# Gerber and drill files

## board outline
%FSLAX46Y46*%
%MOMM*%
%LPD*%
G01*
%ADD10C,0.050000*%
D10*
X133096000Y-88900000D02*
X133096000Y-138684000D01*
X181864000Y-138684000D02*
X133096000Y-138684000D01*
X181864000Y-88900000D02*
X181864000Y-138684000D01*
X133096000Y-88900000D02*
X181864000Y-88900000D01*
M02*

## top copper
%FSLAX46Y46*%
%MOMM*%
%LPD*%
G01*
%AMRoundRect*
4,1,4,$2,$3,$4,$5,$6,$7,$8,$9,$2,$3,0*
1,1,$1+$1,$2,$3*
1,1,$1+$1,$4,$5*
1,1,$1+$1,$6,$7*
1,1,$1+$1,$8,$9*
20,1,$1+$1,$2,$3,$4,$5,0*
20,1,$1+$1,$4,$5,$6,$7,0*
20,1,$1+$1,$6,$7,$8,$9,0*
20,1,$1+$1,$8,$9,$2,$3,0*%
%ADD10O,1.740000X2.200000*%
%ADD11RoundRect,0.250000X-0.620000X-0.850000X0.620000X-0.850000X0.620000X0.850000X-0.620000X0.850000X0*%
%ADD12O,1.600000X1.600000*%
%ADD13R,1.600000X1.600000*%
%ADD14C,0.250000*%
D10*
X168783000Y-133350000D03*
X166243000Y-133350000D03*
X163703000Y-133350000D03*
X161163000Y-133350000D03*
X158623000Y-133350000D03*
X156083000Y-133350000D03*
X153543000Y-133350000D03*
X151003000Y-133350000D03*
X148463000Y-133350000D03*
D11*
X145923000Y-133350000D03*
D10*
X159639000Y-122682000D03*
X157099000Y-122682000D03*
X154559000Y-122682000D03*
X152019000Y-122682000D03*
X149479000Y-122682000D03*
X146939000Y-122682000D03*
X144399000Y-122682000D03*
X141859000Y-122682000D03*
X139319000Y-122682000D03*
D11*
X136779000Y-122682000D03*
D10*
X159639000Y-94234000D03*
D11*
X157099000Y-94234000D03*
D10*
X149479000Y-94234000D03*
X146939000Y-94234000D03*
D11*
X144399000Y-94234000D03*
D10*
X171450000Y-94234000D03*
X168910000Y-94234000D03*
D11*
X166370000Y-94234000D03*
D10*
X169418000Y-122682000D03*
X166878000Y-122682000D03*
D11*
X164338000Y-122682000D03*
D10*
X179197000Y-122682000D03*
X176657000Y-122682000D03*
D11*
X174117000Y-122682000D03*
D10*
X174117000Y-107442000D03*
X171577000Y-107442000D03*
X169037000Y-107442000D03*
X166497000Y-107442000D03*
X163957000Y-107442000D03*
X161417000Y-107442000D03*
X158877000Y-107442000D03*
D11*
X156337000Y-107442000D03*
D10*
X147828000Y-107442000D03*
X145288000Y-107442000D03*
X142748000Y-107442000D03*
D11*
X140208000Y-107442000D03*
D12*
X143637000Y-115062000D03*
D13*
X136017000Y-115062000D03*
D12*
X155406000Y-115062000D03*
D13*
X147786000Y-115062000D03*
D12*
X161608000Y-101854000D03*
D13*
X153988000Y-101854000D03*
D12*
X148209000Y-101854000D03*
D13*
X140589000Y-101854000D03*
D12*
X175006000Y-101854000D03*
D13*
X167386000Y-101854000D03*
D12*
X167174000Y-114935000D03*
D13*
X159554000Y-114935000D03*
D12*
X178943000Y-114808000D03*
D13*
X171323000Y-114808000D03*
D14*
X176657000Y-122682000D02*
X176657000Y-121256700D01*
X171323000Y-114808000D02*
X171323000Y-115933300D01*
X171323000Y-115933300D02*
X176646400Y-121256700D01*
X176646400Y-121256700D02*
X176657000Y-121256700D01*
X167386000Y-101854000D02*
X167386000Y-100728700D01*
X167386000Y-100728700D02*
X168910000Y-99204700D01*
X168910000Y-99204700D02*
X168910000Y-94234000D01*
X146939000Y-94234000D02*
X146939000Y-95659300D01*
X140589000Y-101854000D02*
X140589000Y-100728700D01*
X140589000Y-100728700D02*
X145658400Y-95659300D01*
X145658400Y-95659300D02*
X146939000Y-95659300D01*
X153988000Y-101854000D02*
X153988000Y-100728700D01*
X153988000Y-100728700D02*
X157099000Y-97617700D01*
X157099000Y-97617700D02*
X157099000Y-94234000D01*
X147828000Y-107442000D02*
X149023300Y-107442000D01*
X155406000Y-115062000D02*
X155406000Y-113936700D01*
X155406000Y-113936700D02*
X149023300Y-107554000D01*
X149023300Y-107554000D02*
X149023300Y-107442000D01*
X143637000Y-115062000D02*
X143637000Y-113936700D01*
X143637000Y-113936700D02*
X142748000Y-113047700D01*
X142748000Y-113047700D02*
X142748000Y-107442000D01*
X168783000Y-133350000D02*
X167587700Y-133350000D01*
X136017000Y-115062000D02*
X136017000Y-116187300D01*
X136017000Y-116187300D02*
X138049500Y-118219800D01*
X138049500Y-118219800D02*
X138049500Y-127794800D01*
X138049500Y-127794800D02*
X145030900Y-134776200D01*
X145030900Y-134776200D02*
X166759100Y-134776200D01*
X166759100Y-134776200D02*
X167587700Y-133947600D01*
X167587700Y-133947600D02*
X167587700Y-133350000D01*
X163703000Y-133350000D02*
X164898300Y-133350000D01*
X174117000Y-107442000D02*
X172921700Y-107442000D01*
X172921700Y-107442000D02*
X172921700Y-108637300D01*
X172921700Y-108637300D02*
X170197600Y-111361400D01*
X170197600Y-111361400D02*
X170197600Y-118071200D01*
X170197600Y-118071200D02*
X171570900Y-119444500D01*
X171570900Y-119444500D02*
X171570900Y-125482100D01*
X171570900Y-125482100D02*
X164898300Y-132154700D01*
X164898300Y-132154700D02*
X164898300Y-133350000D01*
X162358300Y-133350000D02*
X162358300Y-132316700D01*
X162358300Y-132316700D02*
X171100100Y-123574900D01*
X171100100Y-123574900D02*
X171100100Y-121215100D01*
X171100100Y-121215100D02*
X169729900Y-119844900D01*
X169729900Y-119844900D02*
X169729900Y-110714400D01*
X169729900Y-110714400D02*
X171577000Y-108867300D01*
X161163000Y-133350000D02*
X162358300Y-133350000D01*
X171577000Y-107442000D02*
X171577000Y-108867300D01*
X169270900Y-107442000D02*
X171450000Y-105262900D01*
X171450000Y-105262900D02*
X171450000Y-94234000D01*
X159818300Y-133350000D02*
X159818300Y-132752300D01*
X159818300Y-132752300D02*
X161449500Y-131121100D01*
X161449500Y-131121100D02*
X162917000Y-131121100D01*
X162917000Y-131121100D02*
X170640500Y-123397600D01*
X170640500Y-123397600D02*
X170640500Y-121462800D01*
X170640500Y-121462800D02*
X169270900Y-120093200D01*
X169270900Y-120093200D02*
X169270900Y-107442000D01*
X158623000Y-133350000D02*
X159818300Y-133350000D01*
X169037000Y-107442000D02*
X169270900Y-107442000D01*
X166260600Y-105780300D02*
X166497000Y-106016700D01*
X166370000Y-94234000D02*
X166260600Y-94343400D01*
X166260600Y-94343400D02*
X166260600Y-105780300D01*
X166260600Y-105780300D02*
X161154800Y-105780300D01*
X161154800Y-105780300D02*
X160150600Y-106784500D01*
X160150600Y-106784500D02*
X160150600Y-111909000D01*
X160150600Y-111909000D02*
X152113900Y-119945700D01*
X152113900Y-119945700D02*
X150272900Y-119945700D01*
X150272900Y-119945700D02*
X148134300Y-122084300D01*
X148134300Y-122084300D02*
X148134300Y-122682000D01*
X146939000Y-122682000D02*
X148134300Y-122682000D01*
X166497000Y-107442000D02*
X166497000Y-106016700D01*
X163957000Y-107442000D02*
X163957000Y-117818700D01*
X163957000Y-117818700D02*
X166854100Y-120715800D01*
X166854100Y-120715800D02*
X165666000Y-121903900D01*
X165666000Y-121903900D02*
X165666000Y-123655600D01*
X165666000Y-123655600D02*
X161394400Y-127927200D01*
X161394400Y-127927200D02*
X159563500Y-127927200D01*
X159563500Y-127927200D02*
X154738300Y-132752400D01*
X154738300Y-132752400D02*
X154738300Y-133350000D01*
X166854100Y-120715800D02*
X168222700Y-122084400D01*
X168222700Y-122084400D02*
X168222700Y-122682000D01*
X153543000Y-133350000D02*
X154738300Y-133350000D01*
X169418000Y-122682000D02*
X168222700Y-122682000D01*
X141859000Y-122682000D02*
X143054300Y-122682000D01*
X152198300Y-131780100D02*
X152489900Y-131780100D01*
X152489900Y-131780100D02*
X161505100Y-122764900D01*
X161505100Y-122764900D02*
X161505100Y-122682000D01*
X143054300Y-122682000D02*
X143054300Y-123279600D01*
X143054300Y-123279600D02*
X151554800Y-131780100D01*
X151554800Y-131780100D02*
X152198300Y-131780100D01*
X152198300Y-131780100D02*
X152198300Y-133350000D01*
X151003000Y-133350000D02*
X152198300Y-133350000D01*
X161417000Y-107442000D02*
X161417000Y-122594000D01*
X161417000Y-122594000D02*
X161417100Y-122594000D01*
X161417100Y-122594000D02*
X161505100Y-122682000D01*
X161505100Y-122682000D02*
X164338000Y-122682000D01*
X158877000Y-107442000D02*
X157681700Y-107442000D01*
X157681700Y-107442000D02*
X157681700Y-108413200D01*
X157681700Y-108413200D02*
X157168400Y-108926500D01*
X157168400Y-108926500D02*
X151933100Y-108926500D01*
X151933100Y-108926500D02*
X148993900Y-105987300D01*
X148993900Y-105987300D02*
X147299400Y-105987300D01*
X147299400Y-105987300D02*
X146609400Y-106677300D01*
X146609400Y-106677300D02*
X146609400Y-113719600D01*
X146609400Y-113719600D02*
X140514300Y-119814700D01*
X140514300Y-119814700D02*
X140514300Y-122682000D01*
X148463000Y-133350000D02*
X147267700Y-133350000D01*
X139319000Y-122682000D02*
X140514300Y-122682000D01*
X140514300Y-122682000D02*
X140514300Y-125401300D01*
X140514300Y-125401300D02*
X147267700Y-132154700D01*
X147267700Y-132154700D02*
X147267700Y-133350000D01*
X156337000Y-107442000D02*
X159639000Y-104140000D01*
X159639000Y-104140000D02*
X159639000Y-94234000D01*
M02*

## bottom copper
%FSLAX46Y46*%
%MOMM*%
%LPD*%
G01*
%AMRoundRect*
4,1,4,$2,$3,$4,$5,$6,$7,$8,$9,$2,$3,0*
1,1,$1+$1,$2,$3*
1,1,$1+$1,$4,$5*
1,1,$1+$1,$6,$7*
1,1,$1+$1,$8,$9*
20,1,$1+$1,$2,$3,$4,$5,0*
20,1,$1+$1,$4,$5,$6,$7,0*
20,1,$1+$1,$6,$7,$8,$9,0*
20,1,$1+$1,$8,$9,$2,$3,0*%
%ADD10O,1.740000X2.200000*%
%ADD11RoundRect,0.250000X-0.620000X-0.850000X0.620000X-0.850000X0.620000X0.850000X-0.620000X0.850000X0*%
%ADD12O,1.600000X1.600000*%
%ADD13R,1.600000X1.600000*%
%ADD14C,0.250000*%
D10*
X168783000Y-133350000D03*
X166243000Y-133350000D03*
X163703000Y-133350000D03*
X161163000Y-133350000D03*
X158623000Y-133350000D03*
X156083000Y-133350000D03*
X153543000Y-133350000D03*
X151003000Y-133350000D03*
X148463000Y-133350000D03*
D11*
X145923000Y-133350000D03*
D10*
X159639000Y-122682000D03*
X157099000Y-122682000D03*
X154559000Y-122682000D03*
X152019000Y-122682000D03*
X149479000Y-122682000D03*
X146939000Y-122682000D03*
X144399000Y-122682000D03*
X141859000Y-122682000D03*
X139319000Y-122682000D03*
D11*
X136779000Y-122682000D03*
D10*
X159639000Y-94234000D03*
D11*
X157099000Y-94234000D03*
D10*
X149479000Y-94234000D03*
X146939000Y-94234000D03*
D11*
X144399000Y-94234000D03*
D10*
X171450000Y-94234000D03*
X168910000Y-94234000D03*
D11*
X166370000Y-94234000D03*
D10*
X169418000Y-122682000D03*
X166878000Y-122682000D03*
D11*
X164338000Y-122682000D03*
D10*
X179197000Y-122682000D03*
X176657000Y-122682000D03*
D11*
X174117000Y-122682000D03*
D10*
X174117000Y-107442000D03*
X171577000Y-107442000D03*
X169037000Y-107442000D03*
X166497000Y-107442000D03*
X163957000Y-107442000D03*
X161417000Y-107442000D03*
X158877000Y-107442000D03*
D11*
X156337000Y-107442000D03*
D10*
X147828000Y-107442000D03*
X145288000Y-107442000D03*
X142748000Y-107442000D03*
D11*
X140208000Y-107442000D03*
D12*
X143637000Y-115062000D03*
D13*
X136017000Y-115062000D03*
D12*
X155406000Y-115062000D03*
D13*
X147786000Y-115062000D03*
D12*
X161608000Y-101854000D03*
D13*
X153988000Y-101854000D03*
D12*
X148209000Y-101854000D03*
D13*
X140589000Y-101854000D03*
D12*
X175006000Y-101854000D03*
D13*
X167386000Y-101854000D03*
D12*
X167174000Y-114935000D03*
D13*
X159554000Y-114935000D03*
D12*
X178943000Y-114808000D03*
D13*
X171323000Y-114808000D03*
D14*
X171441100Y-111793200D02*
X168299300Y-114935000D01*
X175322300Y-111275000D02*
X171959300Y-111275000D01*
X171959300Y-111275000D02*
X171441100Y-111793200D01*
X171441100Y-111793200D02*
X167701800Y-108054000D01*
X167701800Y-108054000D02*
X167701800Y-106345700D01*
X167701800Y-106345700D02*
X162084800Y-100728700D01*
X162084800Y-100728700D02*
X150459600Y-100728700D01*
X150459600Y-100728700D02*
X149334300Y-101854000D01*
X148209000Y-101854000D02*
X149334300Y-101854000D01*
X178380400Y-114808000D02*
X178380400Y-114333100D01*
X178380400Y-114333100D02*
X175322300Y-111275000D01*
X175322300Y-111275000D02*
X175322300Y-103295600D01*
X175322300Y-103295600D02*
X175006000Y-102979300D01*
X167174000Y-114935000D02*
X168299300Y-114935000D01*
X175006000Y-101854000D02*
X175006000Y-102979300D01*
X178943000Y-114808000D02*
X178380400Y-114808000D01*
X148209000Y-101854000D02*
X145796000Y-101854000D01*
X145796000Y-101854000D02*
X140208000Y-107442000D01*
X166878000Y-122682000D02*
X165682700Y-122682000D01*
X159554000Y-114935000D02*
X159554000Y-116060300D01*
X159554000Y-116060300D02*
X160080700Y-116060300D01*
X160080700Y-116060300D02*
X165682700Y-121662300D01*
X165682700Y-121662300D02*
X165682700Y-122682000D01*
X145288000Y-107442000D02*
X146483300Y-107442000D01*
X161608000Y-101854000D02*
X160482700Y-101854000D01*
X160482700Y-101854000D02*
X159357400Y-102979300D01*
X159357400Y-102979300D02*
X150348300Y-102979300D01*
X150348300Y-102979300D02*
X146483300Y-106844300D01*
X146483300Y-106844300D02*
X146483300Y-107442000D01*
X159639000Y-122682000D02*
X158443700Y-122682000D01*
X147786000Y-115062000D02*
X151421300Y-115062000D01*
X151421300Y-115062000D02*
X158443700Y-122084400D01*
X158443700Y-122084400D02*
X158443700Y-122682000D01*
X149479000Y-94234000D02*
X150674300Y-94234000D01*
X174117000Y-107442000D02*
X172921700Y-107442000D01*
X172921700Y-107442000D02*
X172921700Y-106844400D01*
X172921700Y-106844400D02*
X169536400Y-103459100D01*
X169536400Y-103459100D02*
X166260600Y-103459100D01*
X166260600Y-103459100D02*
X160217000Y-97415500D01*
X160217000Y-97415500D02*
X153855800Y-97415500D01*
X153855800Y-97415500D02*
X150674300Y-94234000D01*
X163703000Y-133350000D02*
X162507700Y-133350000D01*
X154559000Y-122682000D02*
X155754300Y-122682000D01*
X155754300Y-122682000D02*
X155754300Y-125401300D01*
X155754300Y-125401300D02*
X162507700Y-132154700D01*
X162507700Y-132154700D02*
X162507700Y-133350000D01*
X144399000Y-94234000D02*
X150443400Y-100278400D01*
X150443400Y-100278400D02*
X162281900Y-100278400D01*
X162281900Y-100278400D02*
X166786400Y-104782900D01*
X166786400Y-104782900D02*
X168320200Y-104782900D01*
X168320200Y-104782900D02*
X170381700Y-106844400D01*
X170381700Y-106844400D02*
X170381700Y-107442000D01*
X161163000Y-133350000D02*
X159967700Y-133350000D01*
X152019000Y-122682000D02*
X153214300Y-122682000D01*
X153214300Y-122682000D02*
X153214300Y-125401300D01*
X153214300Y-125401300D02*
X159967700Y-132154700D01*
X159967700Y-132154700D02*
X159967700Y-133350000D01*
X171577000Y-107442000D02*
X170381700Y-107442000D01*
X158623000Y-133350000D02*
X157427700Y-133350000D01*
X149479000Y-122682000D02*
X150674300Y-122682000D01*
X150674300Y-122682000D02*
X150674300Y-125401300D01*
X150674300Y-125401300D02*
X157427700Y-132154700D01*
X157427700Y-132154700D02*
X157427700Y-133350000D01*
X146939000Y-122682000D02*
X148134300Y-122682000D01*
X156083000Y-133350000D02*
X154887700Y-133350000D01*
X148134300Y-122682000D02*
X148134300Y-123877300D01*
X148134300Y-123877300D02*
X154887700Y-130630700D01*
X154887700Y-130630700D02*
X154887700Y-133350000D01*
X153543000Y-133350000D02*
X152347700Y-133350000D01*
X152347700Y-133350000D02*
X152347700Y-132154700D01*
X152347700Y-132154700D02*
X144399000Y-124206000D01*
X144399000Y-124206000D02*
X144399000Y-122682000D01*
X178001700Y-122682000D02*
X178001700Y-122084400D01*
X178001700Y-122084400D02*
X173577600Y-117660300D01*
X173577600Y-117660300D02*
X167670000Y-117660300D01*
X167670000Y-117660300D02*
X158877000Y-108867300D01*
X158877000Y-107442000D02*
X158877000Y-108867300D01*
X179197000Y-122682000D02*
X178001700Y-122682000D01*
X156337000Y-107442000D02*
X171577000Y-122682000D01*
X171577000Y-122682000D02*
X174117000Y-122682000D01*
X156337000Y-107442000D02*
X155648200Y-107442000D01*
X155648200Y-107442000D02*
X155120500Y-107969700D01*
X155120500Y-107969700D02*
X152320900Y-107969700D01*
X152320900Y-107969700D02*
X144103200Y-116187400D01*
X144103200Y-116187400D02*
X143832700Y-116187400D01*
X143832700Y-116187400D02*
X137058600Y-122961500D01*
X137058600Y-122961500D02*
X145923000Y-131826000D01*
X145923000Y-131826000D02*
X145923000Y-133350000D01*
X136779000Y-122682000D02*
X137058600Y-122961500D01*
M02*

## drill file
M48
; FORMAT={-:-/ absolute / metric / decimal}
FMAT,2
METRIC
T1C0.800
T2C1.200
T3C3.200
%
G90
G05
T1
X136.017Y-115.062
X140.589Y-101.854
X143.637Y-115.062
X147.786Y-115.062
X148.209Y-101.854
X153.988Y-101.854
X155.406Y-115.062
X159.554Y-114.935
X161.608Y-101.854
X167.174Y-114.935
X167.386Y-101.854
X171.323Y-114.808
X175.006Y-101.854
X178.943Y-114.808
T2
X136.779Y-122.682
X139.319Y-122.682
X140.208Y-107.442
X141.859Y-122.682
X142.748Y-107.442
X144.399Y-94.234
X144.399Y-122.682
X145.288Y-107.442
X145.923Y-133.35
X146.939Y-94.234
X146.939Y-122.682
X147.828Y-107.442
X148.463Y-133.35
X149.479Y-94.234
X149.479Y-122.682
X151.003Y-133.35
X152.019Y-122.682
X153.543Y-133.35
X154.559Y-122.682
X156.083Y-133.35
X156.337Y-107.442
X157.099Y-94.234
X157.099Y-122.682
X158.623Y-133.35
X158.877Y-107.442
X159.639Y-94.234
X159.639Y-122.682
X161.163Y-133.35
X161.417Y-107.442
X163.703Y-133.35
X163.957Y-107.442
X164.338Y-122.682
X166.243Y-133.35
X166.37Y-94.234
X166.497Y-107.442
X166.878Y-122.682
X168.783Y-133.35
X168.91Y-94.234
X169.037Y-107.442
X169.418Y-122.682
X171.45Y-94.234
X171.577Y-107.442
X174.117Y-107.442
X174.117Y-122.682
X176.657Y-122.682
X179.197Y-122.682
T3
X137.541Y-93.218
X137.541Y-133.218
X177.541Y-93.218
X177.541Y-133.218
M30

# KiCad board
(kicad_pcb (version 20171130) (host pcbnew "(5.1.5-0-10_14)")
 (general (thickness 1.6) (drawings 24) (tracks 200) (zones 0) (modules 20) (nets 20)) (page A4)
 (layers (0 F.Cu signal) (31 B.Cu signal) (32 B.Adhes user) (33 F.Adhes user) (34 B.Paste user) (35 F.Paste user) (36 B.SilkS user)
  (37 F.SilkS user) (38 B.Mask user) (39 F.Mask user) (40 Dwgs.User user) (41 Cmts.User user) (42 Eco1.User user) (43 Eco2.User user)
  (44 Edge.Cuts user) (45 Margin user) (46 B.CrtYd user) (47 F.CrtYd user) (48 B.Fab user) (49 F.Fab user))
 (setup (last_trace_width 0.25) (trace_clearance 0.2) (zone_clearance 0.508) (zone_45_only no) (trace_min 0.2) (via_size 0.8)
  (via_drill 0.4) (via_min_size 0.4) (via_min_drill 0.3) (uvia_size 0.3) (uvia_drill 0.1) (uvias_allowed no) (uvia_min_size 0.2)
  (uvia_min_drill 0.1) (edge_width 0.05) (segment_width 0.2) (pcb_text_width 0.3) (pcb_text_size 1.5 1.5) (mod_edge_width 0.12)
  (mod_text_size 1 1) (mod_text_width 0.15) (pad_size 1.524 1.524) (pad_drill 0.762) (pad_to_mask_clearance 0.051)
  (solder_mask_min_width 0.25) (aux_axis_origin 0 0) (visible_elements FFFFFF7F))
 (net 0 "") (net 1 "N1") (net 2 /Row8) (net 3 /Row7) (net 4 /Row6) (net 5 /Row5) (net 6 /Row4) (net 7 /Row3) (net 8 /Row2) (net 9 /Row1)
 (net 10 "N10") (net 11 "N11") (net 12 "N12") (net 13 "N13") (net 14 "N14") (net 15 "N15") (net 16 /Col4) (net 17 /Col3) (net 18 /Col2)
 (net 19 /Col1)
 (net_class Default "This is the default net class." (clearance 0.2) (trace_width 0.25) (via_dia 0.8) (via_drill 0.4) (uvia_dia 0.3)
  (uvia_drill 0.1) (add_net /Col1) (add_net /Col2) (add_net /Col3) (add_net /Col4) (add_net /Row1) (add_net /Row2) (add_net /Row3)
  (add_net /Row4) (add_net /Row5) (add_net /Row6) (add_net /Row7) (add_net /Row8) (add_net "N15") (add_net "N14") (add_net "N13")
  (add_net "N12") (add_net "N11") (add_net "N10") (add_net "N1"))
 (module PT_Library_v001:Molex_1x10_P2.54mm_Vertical (layer F.Cu) (at 145.923 133.35)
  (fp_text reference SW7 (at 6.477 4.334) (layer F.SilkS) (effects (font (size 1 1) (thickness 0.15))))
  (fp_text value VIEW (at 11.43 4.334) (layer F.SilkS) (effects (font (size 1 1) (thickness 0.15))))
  (pad 10 thru_hole oval (at 22.86 0) (size 1.74 2.2) (drill 1.2) (layers *.Cu *.Mask) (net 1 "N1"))
  (pad 9 thru_hole oval (at 20.32 0) (size 1.74 2.2) (drill 1.2) (layers *.Cu *.Mask))
  (pad 8 thru_hole oval (at 17.78 0) (size 1.74 2.2) (drill 1.2) (layers *.Cu *.Mask) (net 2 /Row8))
  (pad 7 thru_hole oval (at 15.24 0) (size 1.74 2.2) (drill 1.2) (layers *.Cu *.Mask) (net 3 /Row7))
  (pad 6 thru_hole oval (at 12.7 0) (size 1.74 2.2) (drill 1.2) (layers *.Cu *.Mask) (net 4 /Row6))
  (pad 5 thru_hole oval (at 10.16 0) (size 1.74 2.2) (drill 1.2) (layers *.Cu *.Mask) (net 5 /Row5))
  (pad 4 thru_hole oval (at 7.62 0) (size 1.74 2.2) (drill 1.2) (layers *.Cu *.Mask) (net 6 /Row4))
  (pad 3 thru_hole oval (at 5.08 0) (size 1.74 2.2) (drill 1.2) (layers *.Cu *.Mask) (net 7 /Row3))
  (pad 2 thru_hole oval (at 2.54 0) (size 1.74 2.2) (drill 1.2) (layers *.Cu *.Mask) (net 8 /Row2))
  (pad 1 thru_hole roundrect (at 0 0) (size 1.74 2.2) (drill 1.2) (layers *.Cu *.Mask) (roundrect_rratio 0.143678) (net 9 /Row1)))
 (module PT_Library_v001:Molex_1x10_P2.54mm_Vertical (layer F.Cu) (at 136.779 122.682)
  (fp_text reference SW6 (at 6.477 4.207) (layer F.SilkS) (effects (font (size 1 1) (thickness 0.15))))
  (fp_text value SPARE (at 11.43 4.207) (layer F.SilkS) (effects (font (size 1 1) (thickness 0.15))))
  (pad 10 thru_hole oval (at 22.86 0) (size 1.74 2.2) (drill 1.2) (layers *.Cu *.Mask) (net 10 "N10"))
  (pad 9 thru_hole oval (at 20.32 0) (size 1.74 2.2) (drill 1.2) (layers *.Cu *.Mask))
  (pad 8 thru_hole oval (at 17.78 0) (size 1.74 2.2) (drill 1.2) (layers *.Cu *.Mask) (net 2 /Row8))
  (pad 7 thru_hole oval (at 15.24 0) (size 1.74 2.2) (drill 1.2) (layers *.Cu *.Mask) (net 3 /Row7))
  (pad 6 thru_hole oval (at 12.7 0) (size 1.74 2.2) (drill 1.2) (layers *.Cu *.Mask) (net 4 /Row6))
  (pad 5 thru_hole oval (at 10.16 0) (size 1.74 2.2) (drill 1.2) (layers *.Cu *.Mask) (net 5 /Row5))
  (pad 4 thru_hole oval (at 7.62 0) (size 1.74 2.2) (drill 1.2) (layers *.Cu *.Mask) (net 6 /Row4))
  (pad 3 thru_hole oval (at 5.08 0) (size 1.74 2.2) (drill 1.2) (layers *.Cu *.Mask) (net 7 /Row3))
  (pad 2 thru_hole oval (at 2.54 0) (size 1.74 2.2) (drill 1.2) (layers *.Cu *.Mask) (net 8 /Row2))
  (pad 1 thru_hole roundrect (at 0 0) (size 1.74 2.2) (drill 1.2) (layers *.Cu *.Mask) (roundrect_rratio 0.143678) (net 9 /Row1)))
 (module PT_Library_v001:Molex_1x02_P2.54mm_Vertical (layer F.Cu) (at 157.099 94.234)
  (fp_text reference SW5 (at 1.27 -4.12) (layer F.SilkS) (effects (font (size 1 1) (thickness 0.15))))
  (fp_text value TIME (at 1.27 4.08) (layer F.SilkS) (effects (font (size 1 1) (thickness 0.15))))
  (pad 2 thru_hole oval (at 2.54 0) (size 1.74 2.2) (drill 1.2) (layers *.Cu *.Mask) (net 9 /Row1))
  (pad 1 thru_hole roundrect (at 0 0) (size 1.74 2.2) (drill 1.2) (layers *.Cu *.Mask) (roundrect_rratio 0.143678) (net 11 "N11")))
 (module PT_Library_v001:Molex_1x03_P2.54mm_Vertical (layer F.Cu) (at 144.399 94.234)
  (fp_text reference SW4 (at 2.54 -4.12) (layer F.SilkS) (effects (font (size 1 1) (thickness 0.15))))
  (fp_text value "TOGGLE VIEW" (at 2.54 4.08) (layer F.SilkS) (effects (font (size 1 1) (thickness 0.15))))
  (pad 3 thru_hole oval (at 5.08 0) (size 1.74 2.2) (drill 1.2) (layers *.Cu *.Mask) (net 2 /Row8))
  (pad 2 thru_hole oval (at 2.54 0) (size 1.74 2.2) (drill 1.2) (layers *.Cu *.Mask) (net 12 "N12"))
  (pad 1 thru_hole roundrect (at 0 0) (size 1.74 2.2) (drill 1.2) (layers *.Cu *.Mask) (roundrect_rratio 0.143678) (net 3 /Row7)))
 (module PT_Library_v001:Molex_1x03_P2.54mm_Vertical (layer F.Cu) (at 166.37 94.234)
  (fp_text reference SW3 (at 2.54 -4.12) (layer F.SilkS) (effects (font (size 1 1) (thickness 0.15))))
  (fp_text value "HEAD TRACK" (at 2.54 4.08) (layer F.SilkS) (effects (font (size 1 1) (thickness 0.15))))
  (pad 3 thru_hole oval (at 5.08 0) (size 1.74 2.2) (drill 1.2) (layers *.Cu *.Mask) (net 4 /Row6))
  (pad 2 thru_hole oval (at 2.54 0) (size 1.74 2.2) (drill 1.2) (layers *.Cu *.Mask) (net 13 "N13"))
  (pad 1 thru_hole roundrect (at 0 0) (size 1.74 2.2) (drill 1.2) (layers *.Cu *.Mask) (roundrect_rratio 0.143678) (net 5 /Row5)))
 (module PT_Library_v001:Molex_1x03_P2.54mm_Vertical (layer F.Cu) (at 164.338 122.682)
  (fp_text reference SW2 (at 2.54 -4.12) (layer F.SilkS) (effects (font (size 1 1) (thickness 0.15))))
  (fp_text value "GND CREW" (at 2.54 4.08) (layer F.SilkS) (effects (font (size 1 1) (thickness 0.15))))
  (pad 3 thru_hole oval (at 5.08 0) (size 1.74 2.2) (drill 1.2) (layers *.Cu *.Mask) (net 6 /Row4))
  (pad 2 thru_hole oval (at 2.54 0) (size 1.74 2.2) (drill 1.2) (layers *.Cu *.Mask) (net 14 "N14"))
  (pad 1 thru_hole roundrect (at 0 0) (size 1.74 2.2) (drill 1.2) (layers *.Cu *.Mask) (roundrect_rratio 0.143678) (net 7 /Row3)))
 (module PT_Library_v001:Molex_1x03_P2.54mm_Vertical (layer F.Cu) (at 174.117 122.682)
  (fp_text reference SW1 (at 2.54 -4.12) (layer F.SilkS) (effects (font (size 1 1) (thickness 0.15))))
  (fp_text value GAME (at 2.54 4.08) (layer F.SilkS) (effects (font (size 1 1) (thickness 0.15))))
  (pad 3 thru_hole oval (at 5.08 0) (size 1.74 2.2) (drill 1.2) (layers *.Cu *.Mask) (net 8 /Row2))
  (pad 2 thru_hole oval (at 2.54 0) (size 1.74 2.2) (drill 1.2) (layers *.Cu *.Mask) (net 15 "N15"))
  (pad 1 thru_hole roundrect (at 0 0) (size 1.74 2.2) (drill 1.2) (layers *.Cu *.Mask) (roundrect_rratio 0.143678) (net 9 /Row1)))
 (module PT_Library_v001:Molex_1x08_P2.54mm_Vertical (layer F.Cu) (at 156.337 107.442)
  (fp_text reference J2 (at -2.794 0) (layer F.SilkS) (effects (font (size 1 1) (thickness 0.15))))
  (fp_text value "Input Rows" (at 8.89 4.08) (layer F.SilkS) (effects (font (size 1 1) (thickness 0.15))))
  (pad 8 thru_hole oval (at 17.78 0) (size 1.74 2.2) (drill 1.2) (layers *.Cu *.Mask) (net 2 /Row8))
  (pad 7 thru_hole oval (at 15.24 0) (size 1.74 2.2) (drill 1.2) (layers *.Cu *.Mask) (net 3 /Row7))
  (pad 6 thru_hole oval (at 12.7 0) (size 1.74 2.2) (drill 1.2) (layers *.Cu *.Mask) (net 4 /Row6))
  (pad 5 thru_hole oval (at 10.16 0) (size 1.74 2.2) (drill 1.2) (layers *.Cu *.Mask) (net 5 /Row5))
  (pad 4 thru_hole oval (at 7.62 0) (size 1.74 2.2) (drill 1.2) (layers *.Cu *.Mask) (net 6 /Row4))
  (pad 3 thru_hole oval (at 5.08 0) (size 1.74 2.2) (drill 1.2) (layers *.Cu *.Mask) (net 7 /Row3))
  (pad 2 thru_hole oval (at 2.54 0) (size 1.74 2.2) (drill 1.2) (layers *.Cu *.Mask) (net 8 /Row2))
  (pad 1 thru_hole roundrect (at 0 0) (size 1.74 2.2) (drill 1.2) (layers *.Cu *.Mask) (roundrect_rratio 0.143678) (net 9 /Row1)))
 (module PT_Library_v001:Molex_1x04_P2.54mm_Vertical (layer F.Cu) (at 140.208 107.442)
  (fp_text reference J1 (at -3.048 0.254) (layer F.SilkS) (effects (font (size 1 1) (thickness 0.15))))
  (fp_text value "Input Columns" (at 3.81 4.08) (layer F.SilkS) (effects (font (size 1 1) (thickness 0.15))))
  (pad 4 thru_hole oval (at 7.62 0) (size 1.74 2.2) (drill 1.2) (layers *.Cu *.Mask) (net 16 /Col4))
  (pad 3 thru_hole oval (at 5.08 0) (size 1.74 2.2) (drill 1.2) (layers *.Cu *.Mask) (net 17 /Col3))
  (pad 2 thru_hole oval (at 2.54 0) (size 1.74 2.2) (drill 1.2) (layers *.Cu *.Mask) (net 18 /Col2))
  (pad 1 thru_hole roundrect (at 0 0) (size 1.74 2.2) (drill 1.2) (layers *.Cu *.Mask) (roundrect_rratio 0.143678) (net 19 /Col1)))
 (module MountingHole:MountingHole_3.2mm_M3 (layer F.Cu) (at 137.541 93.218)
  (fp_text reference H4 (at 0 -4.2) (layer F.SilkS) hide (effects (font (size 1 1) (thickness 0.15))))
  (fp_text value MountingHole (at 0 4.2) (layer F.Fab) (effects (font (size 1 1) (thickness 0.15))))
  (pad 1 np_thru_hole circle (at 0 0) (size 3.2 3.2) (drill 3.2) (layers *.Cu *.Mask)))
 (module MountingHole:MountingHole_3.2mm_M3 (layer F.Cu) (at 177.541 93.218)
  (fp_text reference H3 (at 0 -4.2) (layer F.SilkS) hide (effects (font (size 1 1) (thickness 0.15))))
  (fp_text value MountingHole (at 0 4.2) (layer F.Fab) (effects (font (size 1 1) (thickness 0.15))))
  (pad 1 np_thru_hole circle (at 0 0) (size 3.2 3.2) (drill 3.2) (layers *.Cu *.Mask)))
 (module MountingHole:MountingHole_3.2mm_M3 (layer F.Cu) (at 137.541 133.218)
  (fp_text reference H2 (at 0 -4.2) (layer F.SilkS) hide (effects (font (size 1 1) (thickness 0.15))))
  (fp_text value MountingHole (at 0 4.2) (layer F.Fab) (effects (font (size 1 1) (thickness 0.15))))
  (pad 1 np_thru_hole circle (at 0 0) (size 3.2 3.2) (drill 3.2) (layers *.Cu *.Mask)))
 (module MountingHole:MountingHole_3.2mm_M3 (layer F.Cu) (at 177.541 133.218)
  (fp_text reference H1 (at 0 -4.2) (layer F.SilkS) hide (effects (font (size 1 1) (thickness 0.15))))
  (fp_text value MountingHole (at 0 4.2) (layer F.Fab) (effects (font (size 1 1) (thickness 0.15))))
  (pad 1 np_thru_hole circle (at 0 0) (size 3.2 3.2) (drill 3.2) (layers *.Cu *.Mask)))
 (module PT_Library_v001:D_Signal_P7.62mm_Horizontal (layer F.Cu) (at 136.017 115.062)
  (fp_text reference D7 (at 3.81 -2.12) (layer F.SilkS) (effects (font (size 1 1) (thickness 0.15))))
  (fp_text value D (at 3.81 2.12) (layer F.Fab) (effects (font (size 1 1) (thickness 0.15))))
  (pad 2 thru_hole oval (at 7.62 0) (size 1.6 1.6) (drill 0.8) (layers *.Cu *.Mask) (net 18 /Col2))
  (pad 1 thru_hole rect (at 0 0) (size 1.6 1.6) (drill 0.8) (layers *.Cu *.Mask) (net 1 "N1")))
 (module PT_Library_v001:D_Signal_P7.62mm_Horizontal (layer F.Cu) (at 147.786 115.062)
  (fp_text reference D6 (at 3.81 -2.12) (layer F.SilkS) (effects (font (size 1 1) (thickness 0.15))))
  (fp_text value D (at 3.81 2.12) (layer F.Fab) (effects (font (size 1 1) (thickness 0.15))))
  (pad 2 thru_hole oval (at 7.62 0) (size 1.6 1.6) (drill 0.8) (layers *.Cu *.Mask) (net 16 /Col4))
  (pad 1 thru_hole rect (at 0 0) (size 1.6 1.6) (drill 0.8) (layers *.Cu *.Mask) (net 10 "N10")))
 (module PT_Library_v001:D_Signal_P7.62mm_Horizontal (layer F.Cu) (at 153.988 101.854)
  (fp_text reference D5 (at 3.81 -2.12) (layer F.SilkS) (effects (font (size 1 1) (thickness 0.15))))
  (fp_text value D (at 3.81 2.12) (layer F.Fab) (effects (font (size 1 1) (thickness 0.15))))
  (pad 2 thru_hole oval (at 7.62 0) (size 1.6 1.6) (drill 0.8) (layers *.Cu *.Mask) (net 17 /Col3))
  (pad 1 thru_hole rect (at 0 0) (size 1.6 1.6) (drill 0.8) (layers *.Cu *.Mask) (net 11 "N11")))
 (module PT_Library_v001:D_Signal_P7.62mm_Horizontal (layer F.Cu) (at 140.589 101.854)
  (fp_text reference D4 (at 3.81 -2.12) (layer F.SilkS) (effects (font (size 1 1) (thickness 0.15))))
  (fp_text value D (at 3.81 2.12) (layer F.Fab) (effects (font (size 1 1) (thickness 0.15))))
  (pad 2 thru_hole oval (at 7.62 0) (size 1.6 1.6) (drill 0.8) (layers *.Cu *.Mask) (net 19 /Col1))
  (pad 1 thru_hole rect (at 0 0) (size 1.6 1.6) (drill 0.8) (layers *.Cu *.Mask) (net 12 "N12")))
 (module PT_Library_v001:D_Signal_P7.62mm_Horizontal (layer F.Cu) (at 167.386 101.854)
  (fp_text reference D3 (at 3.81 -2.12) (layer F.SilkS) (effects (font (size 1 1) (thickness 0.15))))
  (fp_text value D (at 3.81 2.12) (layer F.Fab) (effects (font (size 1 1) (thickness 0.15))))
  (pad 2 thru_hole oval (at 7.62 0) (size 1.6 1.6) (drill 0.8) (layers *.Cu *.Mask) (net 19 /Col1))
  (pad 1 thru_hole rect (at 0 0) (size 1.6 1.6) (drill 0.8) (layers *.Cu *.Mask) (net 13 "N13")))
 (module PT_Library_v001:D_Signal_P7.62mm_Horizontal (layer F.Cu) (at 159.554 114.935)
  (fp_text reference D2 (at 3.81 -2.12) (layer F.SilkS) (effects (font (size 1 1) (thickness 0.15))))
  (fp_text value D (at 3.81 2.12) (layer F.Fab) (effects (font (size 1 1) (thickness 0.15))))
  (pad 2 thru_hole oval (at 7.62 0) (size 1.6 1.6) (drill 0.8) (layers *.Cu *.Mask) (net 19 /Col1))
  (pad 1 thru_hole rect (at 0 0) (size 1.6 1.6) (drill 0.8) (layers *.Cu *.Mask) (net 14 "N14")))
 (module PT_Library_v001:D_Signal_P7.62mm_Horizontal (layer F.Cu) (at 171.323 114.808)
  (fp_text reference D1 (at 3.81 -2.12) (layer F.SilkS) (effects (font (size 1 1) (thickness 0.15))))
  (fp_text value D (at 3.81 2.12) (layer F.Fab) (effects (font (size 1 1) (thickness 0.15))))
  (pad 2 thru_hole oval (at 7.62 0) (size 1.6 1.6) (drill 0.8) (layers *.Cu *.Mask) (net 19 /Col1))
  (pad 1 thru_hole rect (at 0 0) (size 1.6 1.6) (drill 0.8) (layers *.Cu *.Mask) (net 15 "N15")))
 (gr_line (start 133.096 88.9) (end 133.096 138.684) (layer Edge.Cuts) (width 0.05))
 (gr_line (start 181.864 138.684) (end 133.096 138.684) (layer Edge.Cuts) (width 0.05))
 (gr_line (start 181.864 88.9) (end 181.864 138.684) (layer Edge.Cuts) (width 0.05))
 (gr_line (start 133.096 88.9) (end 181.864 88.9) (layer Edge.Cuts) (width 0.05))
 (segment (start 171.4411 111.7932) (end 168.2993 114.935) (width 0.25) (layer B.Cu) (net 19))
 (segment (start 175.3223 111.275) (end 171.9593 111.275) (width 0.25) (layer B.Cu) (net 19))
 (segment (start 171.9593 111.275) (end 171.4411 111.7932) (width 0.25) (layer B.Cu) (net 19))
 (segment (start 171.4411 111.7932) (end 167.7018 108.054) (width 0.25) (layer B.Cu) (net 19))
 (segment (start 167.7018 108.054) (end 167.7018 106.3457) (width 0.25) (layer B.Cu) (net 19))
 (segment (start 167.7018 106.3457) (end 162.0848 100.7287) (width 0.25) (layer B.Cu) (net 19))
 (segment (start 162.0848 100.7287) (end 150.4596 100.7287) (width 0.25) (layer B.Cu) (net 19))
 (segment (start 150.4596 100.7287) (end 149.3343 101.854) (width 0.25) (layer B.Cu) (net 19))
 (segment (start 148.209 101.854) (end 149.3343 101.854) (width 0.25) (layer B.Cu) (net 19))
 (segment (start 178.3804 114.808) (end 178.3804 114.3331) (width 0.25) (layer B.Cu) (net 19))
 (segment (start 178.3804 114.3331) (end 175.3223 111.275) (width 0.25) (layer B.Cu) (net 19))
 (segment (start 175.3223 111.275) (end 175.3223 103.2956) (width 0.25) (layer B.Cu) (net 19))
 (segment (start 175.3223 103.2956) (end 175.006 102.9793) (width 0.25) (layer B.Cu) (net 19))
 (segment (start 167.174 114.935) (end 168.2993 114.935) (width 0.25) (layer B.Cu) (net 19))
 (segment (start 175.006 101.854) (end 175.006 102.9793) (width 0.25) (layer B.Cu) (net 19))
 (segment (start 178.943 114.808) (end 178.3804 114.808) (width 0.25) (layer B.Cu) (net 19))
 (segment (start 148.209 101.854) (end 145.796 101.854) (width 0.25) (layer B.Cu) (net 19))
 (segment (start 145.796 101.854) (end 140.208 107.442) (width 0.25) (layer B.Cu) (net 19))
 (segment (start 176.657 122.682) (end 176.657 121.2567) (width 0.25) (layer F.Cu) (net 15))
 (segment (start 171.323 114.808) (end 171.323 115.9333) (width 0.25) (layer F.Cu) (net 15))
 (segment (start 171.323 115.9333) (end 176.6464 121.2567) (width 0.25) (layer F.Cu) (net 15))
 (segment (start 176.6464 121.2567) (end 176.657 121.2567) (width 0.25) (layer F.Cu) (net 15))
 (segment (start 166.878 122.682) (end 165.6827 122.682) (width 0.25) (layer B.Cu) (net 14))
 (segment (start 159.554 114.935) (end 159.554 116.0603) (width 0.25) (layer B.Cu) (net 14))
 (segment (start 159.554 116.0603) (end 160.0807 116.0603) (width 0.25) (layer B.Cu) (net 14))
 (segment (start 160.0807 116.0603) (end 165.6827 121.6623) (width 0.25) (layer B.Cu) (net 14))
 (segment (start 165.6827 121.6623) (end 165.6827 122.682) (width 0.25) (layer B.Cu) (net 14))
 (segment (start 167.386 101.854) (end 167.386 100.7287) (width 0.25) (layer F.Cu) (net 13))
 (segment (start 167.386 100.7287) (end 168.91 99.2047) (width 0.25) (layer F.Cu) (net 13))
 (segment (start 168.91 99.2047) (end 168.91 94.234) (width 0.25) (layer F.Cu) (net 13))
 (segment (start 146.939 94.234) (end 146.939 95.6593) (width 0.25) (layer F.Cu) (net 12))
 (segment (start 140.589 101.854) (end 140.589 100.7287) (width 0.25) (layer F.Cu) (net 12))
 (segment (start 140.589 100.7287) (end 145.6584 95.6593) (width 0.25) (layer F.Cu) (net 12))
 (segment (start 145.6584 95.6593) (end 146.939 95.6593) (width 0.25) (layer F.Cu) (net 12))
 (segment (start 145.288 107.442) (end 146.4833 107.442) (width 0.25) (layer B.Cu) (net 17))
 (segment (start 161.608 101.854) (end 160.4827 101.854) (width 0.25) (layer B.Cu) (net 17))
 (segment (start 160.4827 101.854) (end 159.3574 102.9793) (width 0.25) (layer B.Cu) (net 17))
 (segment (start 159.3574 102.9793) (end 150.3483 102.9793) (width 0.25) (layer B.Cu) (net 17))
 (segment (start 150.3483 102.9793) (end 146.4833 106.8443) (width 0.25) (layer B.Cu) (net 17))
 (segment (start 146.4833 106.8443) (end 146.4833 107.442) (width 0.25) (layer B.Cu) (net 17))
 (segment (start 153.988 101.854) (end 153.988 100.7287) (width 0.25) (layer F.Cu) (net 11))
 (segment (start 153.988 100.7287) (end 157.099 97.6177) (width 0.25) (layer F.Cu) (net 11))
 (segment (start 157.099 97.6177) (end 157.099 94.234) (width 0.25) (layer F.Cu) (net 11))
 (segment (start 147.828 107.442) (end 149.0233 107.442) (width 0.25) (layer F.Cu) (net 16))
 (segment (start 155.406 115.062) (end 155.406 113.9367) (width 0.25) (layer F.Cu) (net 16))
 (segment (start 155.406 113.9367) (end 149.0233 107.554) (width 0.25) (layer F.Cu) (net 16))
 (segment (start 149.0233 107.554) (end 149.0233 107.442) (width 0.25) (layer F.Cu) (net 16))
 (segment (start 159.639 122.682) (end 158.4437 122.682) (width 0.25) (layer B.Cu) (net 10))
 (segment (start 147.786 115.062) (end 151.4213 115.062) (width 0.25) (layer B.Cu) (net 10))
 (segment (start 151.4213 115.062) (end 158.4437 122.0844) (width 0.25) (layer B.Cu) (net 10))
 (segment (start 158.4437 122.0844) (end 158.4437 122.682) (width 0.25) (layer B.Cu) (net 10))
 (segment (start 143.637 115.062) (end 143.637 113.9367) (width 0.25) (layer F.Cu) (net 18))
 (segment (start 143.637 113.9367) (end 142.748 113.0477) (width 0.25) (layer F.Cu) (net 18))
 (segment (start 142.748 113.0477) (end 142.748 107.442) (width 0.25) (layer F.Cu) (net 18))
 (segment (start 168.783 133.35) (end 167.5877 133.35) (width 0.25) (layer F.Cu) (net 1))
 (segment (start 136.017 115.062) (end 136.017 116.1873) (width 0.25) (layer F.Cu) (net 1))
 (segment (start 136.017 116.1873) (end 138.0495 118.2198) (width 0.25) (layer F.Cu) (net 1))
 (segment (start 138.0495 118.2198) (end 138.0495 127.7948) (width 0.25) (layer F.Cu) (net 1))
 (segment (start 138.0495 127.7948) (end 145.0309 134.7762) (width 0.25) (layer F.Cu) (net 1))
 (segment (start 145.0309 134.7762) (end 166.7591 134.7762) (width 0.25) (layer F.Cu) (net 1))
 (segment (start 166.7591 134.7762) (end 167.5877 133.9476) (width 0.25) (layer F.Cu) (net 1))
 (segment (start 167.5877 133.9476) (end 167.5877 133.35) (width 0.25) (layer F.Cu) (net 1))
 (segment (start 163.703 133.35) (end 164.8983 133.35) (width 0.25) (layer F.Cu) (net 2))
 (segment (start 174.117 107.442) (end 172.9217 107.442) (width 0.25) (layer F.Cu) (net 2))
 (segment (start 172.9217 107.442) (end 172.9217 108.6373) (width 0.25) (layer F.Cu) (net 2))
 (segment (start 172.9217 108.6373) (end 170.1976 111.3614) (width 0.25) (layer F.Cu) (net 2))
 (segment (start 170.1976 111.3614) (end 170.1976 118.0712) (width 0.25) (layer F.Cu) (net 2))
 (segment (start 170.1976 118.0712) (end 171.5709 119.4445) (width 0.25) (layer F.Cu) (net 2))
 (segment (start 171.5709 119.4445) (end 171.5709 125.4821) (width 0.25) (layer F.Cu) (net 2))
 (segment (start 171.5709 125.4821) (end 164.8983 132.1547) (width 0.25) (layer F.Cu) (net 2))
 (segment (start 164.8983 132.1547) (end 164.8983 133.35) (width 0.25) (layer F.Cu) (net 2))
 (segment (start 149.479 94.234) (end 150.6743 94.234) (width 0.25) (layer B.Cu) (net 2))
 (segment (start 174.117 107.442) (end 172.9217 107.442) (width 0.25) (layer B.Cu) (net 2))
 (segment (start 172.9217 107.442) (end 172.9217 106.8444) (width 0.25) (layer B.Cu) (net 2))
 (segment (start 172.9217 106.8444) (end 169.5364 103.4591) (width 0.25) (layer B.Cu) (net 2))
 (segment (start 169.5364 103.4591) (end 166.2606 103.4591) (width 0.25) (layer B.Cu) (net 2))
 (segment (start 166.2606 103.4591) (end 160.217 97.4155) (width 0.25) (layer B.Cu) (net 2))
 (segment (start 160.217 97.4155) (end 153.8558 97.4155) (width 0.25) (layer B.Cu) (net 2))
 (segment (start 153.8558 97.4155) (end 150.6743 94.234) (width 0.25) (layer B.Cu) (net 2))
 (segment (start 163.703 133.35) (end 162.5077 133.35) (width 0.25) (layer B.Cu) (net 2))
 (segment (start 154.559 122.682) (end 155.7543 122.682) (width 0.25) (layer B.Cu) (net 2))
 (segment (start 155.7543 122.682) (end 155.7543 125.4013) (width 0.25) (layer B.Cu) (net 2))
 (segment (start 155.7543 125.4013) (end 162.5077 132.1547) (width 0.25) (layer B.Cu) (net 2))
 (segment (start 162.5077 132.1547) (end 162.5077 133.35) (width 0.25) (layer B.Cu) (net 2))
 (segment (start 162.3583 133.35) (end 162.3583 132.3167) (width 0.25) (layer F.Cu) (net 3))
 (segment (start 162.3583 132.3167) (end 171.1001 123.5749) (width 0.25) (layer F.Cu) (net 3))
 (segment (start 171.1001 123.5749) (end 171.1001 121.2151) (width 0.25) (layer F.Cu) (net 3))
 (segment (start 171.1001 121.2151) (end 169.7299 119.8449) (width 0.25) (layer F.Cu) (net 3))
 (segment (start 169.7299 119.8449) (end 169.7299 110.7144) (width 0.25) (layer F.Cu) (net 3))
 (segment (start 169.7299 110.7144) (end 171.577 108.8673) (width 0.25) (layer F.Cu) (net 3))
 (segment (start 161.163 133.35) (end 162.3583 133.35) (width 0.25) (layer F.Cu) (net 3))
 (segment (start 171.577 107.442) (end 171.577 108.8673) (width 0.25) (layer F.Cu) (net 3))
 (segment (start 144.399 94.234) (end 150.4434 100.2784) (width 0.25) (layer B.Cu) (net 3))
 (segment (start 150.4434 100.2784) (end 162.2819 100.2784) (width 0.25) (layer B.Cu) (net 3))
 (segment (start 162.2819 100.2784) (end 166.7864 104.7829) (width 0.25) (layer B.Cu) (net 3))
 (segment (start 166.7864 104.7829) (end 168.3202 104.7829) (width 0.25) (layer B.Cu) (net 3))
 (segment (start 168.3202 104.7829) (end 170.3817 106.8444) (width 0.25) (layer B.Cu) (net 3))
 (segment (start 170.3817 106.8444) (end 170.3817 107.442) (width 0.25) (layer B.Cu) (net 3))
 (segment (start 161.163 133.35) (end 159.9677 133.35) (width 0.25) (layer B.Cu) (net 3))
 (segment (start 152.019 122.682) (end 153.2143 122.682) (width 0.25) (layer B.Cu) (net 3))
 (segment (start 153.2143 122.682) (end 153.2143 125.4013) (width 0.25) (layer B.Cu) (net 3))
 (segment (start 153.2143 125.4013) (end 159.9677 132.1547) (width 0.25) (layer B.Cu) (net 3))
 (segment (start 159.9677 132.1547) (end 159.9677 133.35) (width 0.25) (layer B.Cu) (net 3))
 (segment (start 171.577 107.442) (end 170.3817 107.442) (width 0.25) (layer B.Cu) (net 3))
 (segment (start 169.2709 107.442) (end 171.45 105.2629) (width 0.25) (layer F.Cu) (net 4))
 (segment (start 171.45 105.2629) (end 171.45 94.234) (width 0.25) (layer F.Cu) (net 4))
 (segment (start 159.8183 133.35) (end 159.8183 132.7523) (width 0.25) (layer F.Cu) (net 4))
 (segment (start 159.8183 132.7523) (end 161.4495 131.1211) (width 0.25) (layer F.Cu) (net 4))
 (segment (start 161.4495 131.1211) (end 162.917 131.1211) (width 0.25) (layer F.Cu) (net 4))
 (segment (start 162.917 131.1211) (end 170.6405 123.3976) (width 0.25) (layer F.Cu) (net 4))
 (segment (start 170.6405 123.3976) (end 170.6405 121.4628) (width 0.25) (layer F.Cu) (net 4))
 (segment (start 170.6405 121.4628) (end 169.2709 120.0932) (width 0.25) (layer F.Cu) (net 4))
 (segment (start 169.2709 120.0932) (end 169.2709 107.442) (width 0.25) (layer F.Cu) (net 4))
 (segment (start 158.623 133.35) (end 159.8183 133.35) (width 0.25) (layer F.Cu) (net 4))
 (segment (start 169.037 107.442) (end 169.2709 107.442) (width 0.25) (layer F.Cu) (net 4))
 (segment (start 158.623 133.35) (end 157.4277 133.35) (width 0.25) (layer B.Cu) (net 4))
 (segment (start 149.479 122.682) (end 150.6743 122.682) (width 0.25) (layer B.Cu) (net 4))
 (segment (start 150.6743 122.682) (end 150.6743 125.4013) (width 0.25) (layer B.Cu) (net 4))
 (segment (start 150.6743 125.4013) (end 157.4277 132.1547) (width 0.25) (layer B.Cu) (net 4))
 (segment (start 157.4277 132.1547) (end 157.4277 133.35) (width 0.25) (layer B.Cu) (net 4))
 (segment (start 146.939 122.682) (end 148.1343 122.682) (width 0.25) (layer B.Cu) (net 5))
 (segment (start 156.083 133.35) (end 154.8877 133.35) (width 0.25) (layer B.Cu) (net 5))
 (segment (start 148.1343 122.682) (end 148.1343 123.8773) (width 0.25) (layer B.Cu) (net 5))
 (segment (start 148.1343 123.8773) (end 154.8877 130.6307) (width 0.25) (layer B.Cu) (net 5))
 (segment (start 154.8877 130.6307) (end 154.8877 133.35) (width 0.25) (layer B.Cu) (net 5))
 (segment (start 166.2606 105.7803) (end 166.497 106.0167) (width 0.25) (layer F.Cu) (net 5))
 (segment (start 166.37 94.234) (end 166.2606 94.3434) (width 0.25) (layer F.Cu) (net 5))
 (segment (start 166.2606 94.3434) (end 166.2606 105.7803) (width 0.25) (layer F.Cu) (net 5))
 (segment (start 166.2606 105.7803) (end 161.1548 105.7803) (width 0.25) (layer F.Cu) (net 5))
 (segment (start 161.1548 105.7803) (end 160.1506 106.7845) (width 0.25) (layer F.Cu) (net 5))
 (segment (start 160.1506 106.7845) (end 160.1506 111.909) (width 0.25) (layer F.Cu) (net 5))
 (segment (start 160.1506 111.909) (end 152.1139 119.9457) (width 0.25) (layer F.Cu) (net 5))
 (segment (start 152.1139 119.9457) (end 150.2729 119.9457) (width 0.25) (layer F.Cu) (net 5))
 (segment (start 150.2729 119.9457) (end 148.1343 122.0843) (width 0.25) (layer F.Cu) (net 5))
 (segment (start 148.1343 122.0843) (end 148.1343 122.682) (width 0.25) (layer F.Cu) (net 5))
 (segment (start 146.939 122.682) (end 148.1343 122.682) (width 0.25) (layer F.Cu) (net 5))
 (segment (start 166.497 107.442) (end 166.497 106.0167) (width 0.25) (layer F.Cu) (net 5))
 (segment (start 163.957 107.442) (end 163.957 117.8187) (width 0.25) (layer F.Cu) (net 6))
 (segment (start 163.957 117.8187) (end 166.8541 120.7158) (width 0.25) (layer F.Cu) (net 6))
 (segment (start 166.8541 120.7158) (end 165.666 121.9039) (width 0.25) (layer F.Cu) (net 6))
 (segment (start 165.666 121.9039) (end 165.666 123.6556) (width 0.25) (layer F.Cu) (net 6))
 (segment (start 165.666 123.6556) (end 161.3944 127.9272) (width 0.25) (layer F.Cu) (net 6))
 (segment (start 161.3944 127.9272) (end 159.5635 127.9272) (width 0.25) (layer F.Cu) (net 6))
 (segment (start 159.5635 127.9272) (end 154.7383 132.7524) (width 0.25) (layer F.Cu) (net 6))
 (segment (start 154.7383 132.7524) (end 154.7383 133.35) (width 0.25) (layer F.Cu) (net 6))
 (segment (start 166.8541 120.7158) (end 168.2227 122.0844) (width 0.25) (layer F.Cu) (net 6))
 (segment (start 168.2227 122.0844) (end 168.2227 122.682) (width 0.25) (layer F.Cu) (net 6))
 (segment (start 153.543 133.35) (end 154.7383 133.35) (width 0.25) (layer F.Cu) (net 6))
 (segment (start 169.418 122.682) (end 168.2227 122.682) (width 0.25) (layer F.Cu) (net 6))
 (segment (start 153.543 133.35) (end 152.3477 133.35) (width 0.25) (layer B.Cu) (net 6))
 (segment (start 152.3477 133.35) (end 152.3477 132.1547) (width 0.25) (layer B.Cu) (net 6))
 (segment (start 152.3477 132.1547) (end 144.399 124.206) (width 0.25) (layer B.Cu) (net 6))
 (segment (start 144.399 124.206) (end 144.399 122.682) (width 0.25) (layer B.Cu) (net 6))
 (segment (start 141.859 122.682) (end 143.0543 122.682) (width 0.25) (layer F.Cu) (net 7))
 (segment (start 152.1983 131.7801) (end 152.4899 131.7801) (width 0.25) (layer F.Cu) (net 7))
 (segment (start 152.4899 131.7801) (end 161.5051 122.7649) (width 0.25) (layer F.Cu) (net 7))
 (segment (start 161.5051 122.7649) (end 161.5051 122.682) (width 0.25) (layer F.Cu) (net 7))
 (segment (start 143.0543 122.682) (end 143.0543 123.2796) (width 0.25) (layer F.Cu) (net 7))
 (segment (start 143.0543 123.2796) (end 151.5548 131.7801) (width 0.25) (layer F.Cu) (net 7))
 (segment (start 151.5548 131.7801) (end 152.1983 131.7801) (width 0.25) (layer F.Cu) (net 7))
 (segment (start 152.1983 131.7801) (end 152.1983 133.35) (width 0.25) (layer F.Cu) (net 7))
 (segment (start 151.003 133.35) (end 152.1983 133.35) (width 0.25) (layer F.Cu) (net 7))
 (segment (start 161.417 107.442) (end 161.417 122.594) (width 0.25) (layer F.Cu) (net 7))
 (segment (start 161.417 122.594) (end 161.4171 122.594) (width 0.25) (layer F.Cu) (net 7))
 (segment (start 161.4171 122.594) (end 161.5051 122.682) (width 0.25) (layer F.Cu) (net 7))
 (segment (start 161.5051 122.682) (end 164.338 122.682) (width 0.25) (layer F.Cu) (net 7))
 (segment (start 178.0017 122.682) (end 178.0017 122.0844) (width 0.25) (layer B.Cu) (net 8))
 (segment (start 178.0017 122.0844) (end 173.5776 117.6603) (width 0.25) (layer B.Cu) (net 8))
 (segment (start 173.5776 117.6603) (end 167.67 117.6603) (width 0.25) (layer B.Cu) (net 8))
 (segment (start 167.67 117.6603) (end 158.877 108.8673) (width 0.25) (layer B.Cu) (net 8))
 (segment (start 158.877 107.442) (end 158.877 108.8673) (width 0.25) (layer B.Cu) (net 8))
 (segment (start 179.197 122.682) (end 178.0017 122.682) (width 0.25) (layer B.Cu) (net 8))
 (segment (start 158.877 107.442) (end 157.6817 107.442) (width 0.25) (layer F.Cu) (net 8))
 (segment (start 157.6817 107.442) (end 157.6817 108.4132) (width 0.25) (layer F.Cu) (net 8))
 (segment (start 157.6817 108.4132) (end 157.1684 108.9265) (width 0.25) (layer F.Cu) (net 8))
 (segment (start 157.1684 108.9265) (end 151.9331 108.9265) (width 0.25) (layer F.Cu) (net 8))
 (segment (start 151.9331 108.9265) (end 148.9939 105.9873) (width 0.25) (layer F.Cu) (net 8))
 (segment (start 148.9939 105.9873) (end 147.2994 105.9873) (width 0.25) (layer F.Cu) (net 8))
 (segment (start 147.2994 105.9873) (end 146.6094 106.6773) (width 0.25) (layer F.Cu) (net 8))
 (segment (start 146.6094 106.6773) (end 146.6094 113.7196) (width 0.25) (layer F.Cu) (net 8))
 (segment (start 146.6094 113.7196) (end 140.5143 119.8147) (width 0.25) (layer F.Cu) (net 8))
 (segment (start 140.5143 119.8147) (end 140.5143 122.682) (width 0.25) (layer F.Cu) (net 8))
 (segment (start 148.463 133.35) (end 147.2677 133.35) (width 0.25) (layer F.Cu) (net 8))
 (segment (start 139.319 122.682) (end 140.5143 122.682) (width 0.25) (layer F.Cu) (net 8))
 (segment (start 140.5143 122.682) (end 140.5143 125.4013) (width 0.25) (layer F.Cu) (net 8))
 (segment (start 140.5143 125.4013) (end 147.2677 132.1547) (width 0.25) (layer F.Cu) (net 8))
 (segment (start 147.2677 132.1547) (end 147.2677 133.35) (width 0.25) (layer F.Cu) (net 8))
 (segment (start 156.337 107.442) (end 171.577 122.682) (width 0.25) (layer B.Cu) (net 9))
 (segment (start 171.577 122.682) (end 174.117 122.682) (width 0.25) (layer B.Cu) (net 9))
 (segment (start 156.337 107.442) (end 155.6482 107.442) (width 0.25) (layer B.Cu) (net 9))
 (segment (start 155.6482 107.442) (end 155.1205 107.9697) (width 0.25) (layer B.Cu) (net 9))
 (segment (start 155.1205 107.9697) (end 152.3209 107.9697) (width 0.25) (layer B.Cu) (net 9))
 (segment (start 152.3209 107.9697) (end 144.1032 116.1874) (width 0.25) (layer B.Cu) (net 9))
 (segment (start 144.1032 116.1874) (end 143.8327 116.1874) (width 0.25) (layer B.Cu) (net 9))
 (segment (start 143.8327 116.1874) (end 137.0586 122.9615) (width 0.25) (layer B.Cu) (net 9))
 (segment (start 137.0586 122.9615) (end 145.923 131.826) (width 0.25) (layer B.Cu) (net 9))
 (segment (start 145.923 131.826) (end 145.923 133.35) (width 0.25) (layer B.Cu) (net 9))
 (segment (start 136.779 122.682) (end 137.0586 122.9615) (width 0.25) (layer B.Cu) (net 9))
 (segment (start 156.337 107.442) (end 159.639 104.14) (width 0.25) (layer F.Cu) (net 9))
 (segment (start 159.639 104.14) (end 159.639 94.234) (width 0.25) (layer F.Cu) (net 9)))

